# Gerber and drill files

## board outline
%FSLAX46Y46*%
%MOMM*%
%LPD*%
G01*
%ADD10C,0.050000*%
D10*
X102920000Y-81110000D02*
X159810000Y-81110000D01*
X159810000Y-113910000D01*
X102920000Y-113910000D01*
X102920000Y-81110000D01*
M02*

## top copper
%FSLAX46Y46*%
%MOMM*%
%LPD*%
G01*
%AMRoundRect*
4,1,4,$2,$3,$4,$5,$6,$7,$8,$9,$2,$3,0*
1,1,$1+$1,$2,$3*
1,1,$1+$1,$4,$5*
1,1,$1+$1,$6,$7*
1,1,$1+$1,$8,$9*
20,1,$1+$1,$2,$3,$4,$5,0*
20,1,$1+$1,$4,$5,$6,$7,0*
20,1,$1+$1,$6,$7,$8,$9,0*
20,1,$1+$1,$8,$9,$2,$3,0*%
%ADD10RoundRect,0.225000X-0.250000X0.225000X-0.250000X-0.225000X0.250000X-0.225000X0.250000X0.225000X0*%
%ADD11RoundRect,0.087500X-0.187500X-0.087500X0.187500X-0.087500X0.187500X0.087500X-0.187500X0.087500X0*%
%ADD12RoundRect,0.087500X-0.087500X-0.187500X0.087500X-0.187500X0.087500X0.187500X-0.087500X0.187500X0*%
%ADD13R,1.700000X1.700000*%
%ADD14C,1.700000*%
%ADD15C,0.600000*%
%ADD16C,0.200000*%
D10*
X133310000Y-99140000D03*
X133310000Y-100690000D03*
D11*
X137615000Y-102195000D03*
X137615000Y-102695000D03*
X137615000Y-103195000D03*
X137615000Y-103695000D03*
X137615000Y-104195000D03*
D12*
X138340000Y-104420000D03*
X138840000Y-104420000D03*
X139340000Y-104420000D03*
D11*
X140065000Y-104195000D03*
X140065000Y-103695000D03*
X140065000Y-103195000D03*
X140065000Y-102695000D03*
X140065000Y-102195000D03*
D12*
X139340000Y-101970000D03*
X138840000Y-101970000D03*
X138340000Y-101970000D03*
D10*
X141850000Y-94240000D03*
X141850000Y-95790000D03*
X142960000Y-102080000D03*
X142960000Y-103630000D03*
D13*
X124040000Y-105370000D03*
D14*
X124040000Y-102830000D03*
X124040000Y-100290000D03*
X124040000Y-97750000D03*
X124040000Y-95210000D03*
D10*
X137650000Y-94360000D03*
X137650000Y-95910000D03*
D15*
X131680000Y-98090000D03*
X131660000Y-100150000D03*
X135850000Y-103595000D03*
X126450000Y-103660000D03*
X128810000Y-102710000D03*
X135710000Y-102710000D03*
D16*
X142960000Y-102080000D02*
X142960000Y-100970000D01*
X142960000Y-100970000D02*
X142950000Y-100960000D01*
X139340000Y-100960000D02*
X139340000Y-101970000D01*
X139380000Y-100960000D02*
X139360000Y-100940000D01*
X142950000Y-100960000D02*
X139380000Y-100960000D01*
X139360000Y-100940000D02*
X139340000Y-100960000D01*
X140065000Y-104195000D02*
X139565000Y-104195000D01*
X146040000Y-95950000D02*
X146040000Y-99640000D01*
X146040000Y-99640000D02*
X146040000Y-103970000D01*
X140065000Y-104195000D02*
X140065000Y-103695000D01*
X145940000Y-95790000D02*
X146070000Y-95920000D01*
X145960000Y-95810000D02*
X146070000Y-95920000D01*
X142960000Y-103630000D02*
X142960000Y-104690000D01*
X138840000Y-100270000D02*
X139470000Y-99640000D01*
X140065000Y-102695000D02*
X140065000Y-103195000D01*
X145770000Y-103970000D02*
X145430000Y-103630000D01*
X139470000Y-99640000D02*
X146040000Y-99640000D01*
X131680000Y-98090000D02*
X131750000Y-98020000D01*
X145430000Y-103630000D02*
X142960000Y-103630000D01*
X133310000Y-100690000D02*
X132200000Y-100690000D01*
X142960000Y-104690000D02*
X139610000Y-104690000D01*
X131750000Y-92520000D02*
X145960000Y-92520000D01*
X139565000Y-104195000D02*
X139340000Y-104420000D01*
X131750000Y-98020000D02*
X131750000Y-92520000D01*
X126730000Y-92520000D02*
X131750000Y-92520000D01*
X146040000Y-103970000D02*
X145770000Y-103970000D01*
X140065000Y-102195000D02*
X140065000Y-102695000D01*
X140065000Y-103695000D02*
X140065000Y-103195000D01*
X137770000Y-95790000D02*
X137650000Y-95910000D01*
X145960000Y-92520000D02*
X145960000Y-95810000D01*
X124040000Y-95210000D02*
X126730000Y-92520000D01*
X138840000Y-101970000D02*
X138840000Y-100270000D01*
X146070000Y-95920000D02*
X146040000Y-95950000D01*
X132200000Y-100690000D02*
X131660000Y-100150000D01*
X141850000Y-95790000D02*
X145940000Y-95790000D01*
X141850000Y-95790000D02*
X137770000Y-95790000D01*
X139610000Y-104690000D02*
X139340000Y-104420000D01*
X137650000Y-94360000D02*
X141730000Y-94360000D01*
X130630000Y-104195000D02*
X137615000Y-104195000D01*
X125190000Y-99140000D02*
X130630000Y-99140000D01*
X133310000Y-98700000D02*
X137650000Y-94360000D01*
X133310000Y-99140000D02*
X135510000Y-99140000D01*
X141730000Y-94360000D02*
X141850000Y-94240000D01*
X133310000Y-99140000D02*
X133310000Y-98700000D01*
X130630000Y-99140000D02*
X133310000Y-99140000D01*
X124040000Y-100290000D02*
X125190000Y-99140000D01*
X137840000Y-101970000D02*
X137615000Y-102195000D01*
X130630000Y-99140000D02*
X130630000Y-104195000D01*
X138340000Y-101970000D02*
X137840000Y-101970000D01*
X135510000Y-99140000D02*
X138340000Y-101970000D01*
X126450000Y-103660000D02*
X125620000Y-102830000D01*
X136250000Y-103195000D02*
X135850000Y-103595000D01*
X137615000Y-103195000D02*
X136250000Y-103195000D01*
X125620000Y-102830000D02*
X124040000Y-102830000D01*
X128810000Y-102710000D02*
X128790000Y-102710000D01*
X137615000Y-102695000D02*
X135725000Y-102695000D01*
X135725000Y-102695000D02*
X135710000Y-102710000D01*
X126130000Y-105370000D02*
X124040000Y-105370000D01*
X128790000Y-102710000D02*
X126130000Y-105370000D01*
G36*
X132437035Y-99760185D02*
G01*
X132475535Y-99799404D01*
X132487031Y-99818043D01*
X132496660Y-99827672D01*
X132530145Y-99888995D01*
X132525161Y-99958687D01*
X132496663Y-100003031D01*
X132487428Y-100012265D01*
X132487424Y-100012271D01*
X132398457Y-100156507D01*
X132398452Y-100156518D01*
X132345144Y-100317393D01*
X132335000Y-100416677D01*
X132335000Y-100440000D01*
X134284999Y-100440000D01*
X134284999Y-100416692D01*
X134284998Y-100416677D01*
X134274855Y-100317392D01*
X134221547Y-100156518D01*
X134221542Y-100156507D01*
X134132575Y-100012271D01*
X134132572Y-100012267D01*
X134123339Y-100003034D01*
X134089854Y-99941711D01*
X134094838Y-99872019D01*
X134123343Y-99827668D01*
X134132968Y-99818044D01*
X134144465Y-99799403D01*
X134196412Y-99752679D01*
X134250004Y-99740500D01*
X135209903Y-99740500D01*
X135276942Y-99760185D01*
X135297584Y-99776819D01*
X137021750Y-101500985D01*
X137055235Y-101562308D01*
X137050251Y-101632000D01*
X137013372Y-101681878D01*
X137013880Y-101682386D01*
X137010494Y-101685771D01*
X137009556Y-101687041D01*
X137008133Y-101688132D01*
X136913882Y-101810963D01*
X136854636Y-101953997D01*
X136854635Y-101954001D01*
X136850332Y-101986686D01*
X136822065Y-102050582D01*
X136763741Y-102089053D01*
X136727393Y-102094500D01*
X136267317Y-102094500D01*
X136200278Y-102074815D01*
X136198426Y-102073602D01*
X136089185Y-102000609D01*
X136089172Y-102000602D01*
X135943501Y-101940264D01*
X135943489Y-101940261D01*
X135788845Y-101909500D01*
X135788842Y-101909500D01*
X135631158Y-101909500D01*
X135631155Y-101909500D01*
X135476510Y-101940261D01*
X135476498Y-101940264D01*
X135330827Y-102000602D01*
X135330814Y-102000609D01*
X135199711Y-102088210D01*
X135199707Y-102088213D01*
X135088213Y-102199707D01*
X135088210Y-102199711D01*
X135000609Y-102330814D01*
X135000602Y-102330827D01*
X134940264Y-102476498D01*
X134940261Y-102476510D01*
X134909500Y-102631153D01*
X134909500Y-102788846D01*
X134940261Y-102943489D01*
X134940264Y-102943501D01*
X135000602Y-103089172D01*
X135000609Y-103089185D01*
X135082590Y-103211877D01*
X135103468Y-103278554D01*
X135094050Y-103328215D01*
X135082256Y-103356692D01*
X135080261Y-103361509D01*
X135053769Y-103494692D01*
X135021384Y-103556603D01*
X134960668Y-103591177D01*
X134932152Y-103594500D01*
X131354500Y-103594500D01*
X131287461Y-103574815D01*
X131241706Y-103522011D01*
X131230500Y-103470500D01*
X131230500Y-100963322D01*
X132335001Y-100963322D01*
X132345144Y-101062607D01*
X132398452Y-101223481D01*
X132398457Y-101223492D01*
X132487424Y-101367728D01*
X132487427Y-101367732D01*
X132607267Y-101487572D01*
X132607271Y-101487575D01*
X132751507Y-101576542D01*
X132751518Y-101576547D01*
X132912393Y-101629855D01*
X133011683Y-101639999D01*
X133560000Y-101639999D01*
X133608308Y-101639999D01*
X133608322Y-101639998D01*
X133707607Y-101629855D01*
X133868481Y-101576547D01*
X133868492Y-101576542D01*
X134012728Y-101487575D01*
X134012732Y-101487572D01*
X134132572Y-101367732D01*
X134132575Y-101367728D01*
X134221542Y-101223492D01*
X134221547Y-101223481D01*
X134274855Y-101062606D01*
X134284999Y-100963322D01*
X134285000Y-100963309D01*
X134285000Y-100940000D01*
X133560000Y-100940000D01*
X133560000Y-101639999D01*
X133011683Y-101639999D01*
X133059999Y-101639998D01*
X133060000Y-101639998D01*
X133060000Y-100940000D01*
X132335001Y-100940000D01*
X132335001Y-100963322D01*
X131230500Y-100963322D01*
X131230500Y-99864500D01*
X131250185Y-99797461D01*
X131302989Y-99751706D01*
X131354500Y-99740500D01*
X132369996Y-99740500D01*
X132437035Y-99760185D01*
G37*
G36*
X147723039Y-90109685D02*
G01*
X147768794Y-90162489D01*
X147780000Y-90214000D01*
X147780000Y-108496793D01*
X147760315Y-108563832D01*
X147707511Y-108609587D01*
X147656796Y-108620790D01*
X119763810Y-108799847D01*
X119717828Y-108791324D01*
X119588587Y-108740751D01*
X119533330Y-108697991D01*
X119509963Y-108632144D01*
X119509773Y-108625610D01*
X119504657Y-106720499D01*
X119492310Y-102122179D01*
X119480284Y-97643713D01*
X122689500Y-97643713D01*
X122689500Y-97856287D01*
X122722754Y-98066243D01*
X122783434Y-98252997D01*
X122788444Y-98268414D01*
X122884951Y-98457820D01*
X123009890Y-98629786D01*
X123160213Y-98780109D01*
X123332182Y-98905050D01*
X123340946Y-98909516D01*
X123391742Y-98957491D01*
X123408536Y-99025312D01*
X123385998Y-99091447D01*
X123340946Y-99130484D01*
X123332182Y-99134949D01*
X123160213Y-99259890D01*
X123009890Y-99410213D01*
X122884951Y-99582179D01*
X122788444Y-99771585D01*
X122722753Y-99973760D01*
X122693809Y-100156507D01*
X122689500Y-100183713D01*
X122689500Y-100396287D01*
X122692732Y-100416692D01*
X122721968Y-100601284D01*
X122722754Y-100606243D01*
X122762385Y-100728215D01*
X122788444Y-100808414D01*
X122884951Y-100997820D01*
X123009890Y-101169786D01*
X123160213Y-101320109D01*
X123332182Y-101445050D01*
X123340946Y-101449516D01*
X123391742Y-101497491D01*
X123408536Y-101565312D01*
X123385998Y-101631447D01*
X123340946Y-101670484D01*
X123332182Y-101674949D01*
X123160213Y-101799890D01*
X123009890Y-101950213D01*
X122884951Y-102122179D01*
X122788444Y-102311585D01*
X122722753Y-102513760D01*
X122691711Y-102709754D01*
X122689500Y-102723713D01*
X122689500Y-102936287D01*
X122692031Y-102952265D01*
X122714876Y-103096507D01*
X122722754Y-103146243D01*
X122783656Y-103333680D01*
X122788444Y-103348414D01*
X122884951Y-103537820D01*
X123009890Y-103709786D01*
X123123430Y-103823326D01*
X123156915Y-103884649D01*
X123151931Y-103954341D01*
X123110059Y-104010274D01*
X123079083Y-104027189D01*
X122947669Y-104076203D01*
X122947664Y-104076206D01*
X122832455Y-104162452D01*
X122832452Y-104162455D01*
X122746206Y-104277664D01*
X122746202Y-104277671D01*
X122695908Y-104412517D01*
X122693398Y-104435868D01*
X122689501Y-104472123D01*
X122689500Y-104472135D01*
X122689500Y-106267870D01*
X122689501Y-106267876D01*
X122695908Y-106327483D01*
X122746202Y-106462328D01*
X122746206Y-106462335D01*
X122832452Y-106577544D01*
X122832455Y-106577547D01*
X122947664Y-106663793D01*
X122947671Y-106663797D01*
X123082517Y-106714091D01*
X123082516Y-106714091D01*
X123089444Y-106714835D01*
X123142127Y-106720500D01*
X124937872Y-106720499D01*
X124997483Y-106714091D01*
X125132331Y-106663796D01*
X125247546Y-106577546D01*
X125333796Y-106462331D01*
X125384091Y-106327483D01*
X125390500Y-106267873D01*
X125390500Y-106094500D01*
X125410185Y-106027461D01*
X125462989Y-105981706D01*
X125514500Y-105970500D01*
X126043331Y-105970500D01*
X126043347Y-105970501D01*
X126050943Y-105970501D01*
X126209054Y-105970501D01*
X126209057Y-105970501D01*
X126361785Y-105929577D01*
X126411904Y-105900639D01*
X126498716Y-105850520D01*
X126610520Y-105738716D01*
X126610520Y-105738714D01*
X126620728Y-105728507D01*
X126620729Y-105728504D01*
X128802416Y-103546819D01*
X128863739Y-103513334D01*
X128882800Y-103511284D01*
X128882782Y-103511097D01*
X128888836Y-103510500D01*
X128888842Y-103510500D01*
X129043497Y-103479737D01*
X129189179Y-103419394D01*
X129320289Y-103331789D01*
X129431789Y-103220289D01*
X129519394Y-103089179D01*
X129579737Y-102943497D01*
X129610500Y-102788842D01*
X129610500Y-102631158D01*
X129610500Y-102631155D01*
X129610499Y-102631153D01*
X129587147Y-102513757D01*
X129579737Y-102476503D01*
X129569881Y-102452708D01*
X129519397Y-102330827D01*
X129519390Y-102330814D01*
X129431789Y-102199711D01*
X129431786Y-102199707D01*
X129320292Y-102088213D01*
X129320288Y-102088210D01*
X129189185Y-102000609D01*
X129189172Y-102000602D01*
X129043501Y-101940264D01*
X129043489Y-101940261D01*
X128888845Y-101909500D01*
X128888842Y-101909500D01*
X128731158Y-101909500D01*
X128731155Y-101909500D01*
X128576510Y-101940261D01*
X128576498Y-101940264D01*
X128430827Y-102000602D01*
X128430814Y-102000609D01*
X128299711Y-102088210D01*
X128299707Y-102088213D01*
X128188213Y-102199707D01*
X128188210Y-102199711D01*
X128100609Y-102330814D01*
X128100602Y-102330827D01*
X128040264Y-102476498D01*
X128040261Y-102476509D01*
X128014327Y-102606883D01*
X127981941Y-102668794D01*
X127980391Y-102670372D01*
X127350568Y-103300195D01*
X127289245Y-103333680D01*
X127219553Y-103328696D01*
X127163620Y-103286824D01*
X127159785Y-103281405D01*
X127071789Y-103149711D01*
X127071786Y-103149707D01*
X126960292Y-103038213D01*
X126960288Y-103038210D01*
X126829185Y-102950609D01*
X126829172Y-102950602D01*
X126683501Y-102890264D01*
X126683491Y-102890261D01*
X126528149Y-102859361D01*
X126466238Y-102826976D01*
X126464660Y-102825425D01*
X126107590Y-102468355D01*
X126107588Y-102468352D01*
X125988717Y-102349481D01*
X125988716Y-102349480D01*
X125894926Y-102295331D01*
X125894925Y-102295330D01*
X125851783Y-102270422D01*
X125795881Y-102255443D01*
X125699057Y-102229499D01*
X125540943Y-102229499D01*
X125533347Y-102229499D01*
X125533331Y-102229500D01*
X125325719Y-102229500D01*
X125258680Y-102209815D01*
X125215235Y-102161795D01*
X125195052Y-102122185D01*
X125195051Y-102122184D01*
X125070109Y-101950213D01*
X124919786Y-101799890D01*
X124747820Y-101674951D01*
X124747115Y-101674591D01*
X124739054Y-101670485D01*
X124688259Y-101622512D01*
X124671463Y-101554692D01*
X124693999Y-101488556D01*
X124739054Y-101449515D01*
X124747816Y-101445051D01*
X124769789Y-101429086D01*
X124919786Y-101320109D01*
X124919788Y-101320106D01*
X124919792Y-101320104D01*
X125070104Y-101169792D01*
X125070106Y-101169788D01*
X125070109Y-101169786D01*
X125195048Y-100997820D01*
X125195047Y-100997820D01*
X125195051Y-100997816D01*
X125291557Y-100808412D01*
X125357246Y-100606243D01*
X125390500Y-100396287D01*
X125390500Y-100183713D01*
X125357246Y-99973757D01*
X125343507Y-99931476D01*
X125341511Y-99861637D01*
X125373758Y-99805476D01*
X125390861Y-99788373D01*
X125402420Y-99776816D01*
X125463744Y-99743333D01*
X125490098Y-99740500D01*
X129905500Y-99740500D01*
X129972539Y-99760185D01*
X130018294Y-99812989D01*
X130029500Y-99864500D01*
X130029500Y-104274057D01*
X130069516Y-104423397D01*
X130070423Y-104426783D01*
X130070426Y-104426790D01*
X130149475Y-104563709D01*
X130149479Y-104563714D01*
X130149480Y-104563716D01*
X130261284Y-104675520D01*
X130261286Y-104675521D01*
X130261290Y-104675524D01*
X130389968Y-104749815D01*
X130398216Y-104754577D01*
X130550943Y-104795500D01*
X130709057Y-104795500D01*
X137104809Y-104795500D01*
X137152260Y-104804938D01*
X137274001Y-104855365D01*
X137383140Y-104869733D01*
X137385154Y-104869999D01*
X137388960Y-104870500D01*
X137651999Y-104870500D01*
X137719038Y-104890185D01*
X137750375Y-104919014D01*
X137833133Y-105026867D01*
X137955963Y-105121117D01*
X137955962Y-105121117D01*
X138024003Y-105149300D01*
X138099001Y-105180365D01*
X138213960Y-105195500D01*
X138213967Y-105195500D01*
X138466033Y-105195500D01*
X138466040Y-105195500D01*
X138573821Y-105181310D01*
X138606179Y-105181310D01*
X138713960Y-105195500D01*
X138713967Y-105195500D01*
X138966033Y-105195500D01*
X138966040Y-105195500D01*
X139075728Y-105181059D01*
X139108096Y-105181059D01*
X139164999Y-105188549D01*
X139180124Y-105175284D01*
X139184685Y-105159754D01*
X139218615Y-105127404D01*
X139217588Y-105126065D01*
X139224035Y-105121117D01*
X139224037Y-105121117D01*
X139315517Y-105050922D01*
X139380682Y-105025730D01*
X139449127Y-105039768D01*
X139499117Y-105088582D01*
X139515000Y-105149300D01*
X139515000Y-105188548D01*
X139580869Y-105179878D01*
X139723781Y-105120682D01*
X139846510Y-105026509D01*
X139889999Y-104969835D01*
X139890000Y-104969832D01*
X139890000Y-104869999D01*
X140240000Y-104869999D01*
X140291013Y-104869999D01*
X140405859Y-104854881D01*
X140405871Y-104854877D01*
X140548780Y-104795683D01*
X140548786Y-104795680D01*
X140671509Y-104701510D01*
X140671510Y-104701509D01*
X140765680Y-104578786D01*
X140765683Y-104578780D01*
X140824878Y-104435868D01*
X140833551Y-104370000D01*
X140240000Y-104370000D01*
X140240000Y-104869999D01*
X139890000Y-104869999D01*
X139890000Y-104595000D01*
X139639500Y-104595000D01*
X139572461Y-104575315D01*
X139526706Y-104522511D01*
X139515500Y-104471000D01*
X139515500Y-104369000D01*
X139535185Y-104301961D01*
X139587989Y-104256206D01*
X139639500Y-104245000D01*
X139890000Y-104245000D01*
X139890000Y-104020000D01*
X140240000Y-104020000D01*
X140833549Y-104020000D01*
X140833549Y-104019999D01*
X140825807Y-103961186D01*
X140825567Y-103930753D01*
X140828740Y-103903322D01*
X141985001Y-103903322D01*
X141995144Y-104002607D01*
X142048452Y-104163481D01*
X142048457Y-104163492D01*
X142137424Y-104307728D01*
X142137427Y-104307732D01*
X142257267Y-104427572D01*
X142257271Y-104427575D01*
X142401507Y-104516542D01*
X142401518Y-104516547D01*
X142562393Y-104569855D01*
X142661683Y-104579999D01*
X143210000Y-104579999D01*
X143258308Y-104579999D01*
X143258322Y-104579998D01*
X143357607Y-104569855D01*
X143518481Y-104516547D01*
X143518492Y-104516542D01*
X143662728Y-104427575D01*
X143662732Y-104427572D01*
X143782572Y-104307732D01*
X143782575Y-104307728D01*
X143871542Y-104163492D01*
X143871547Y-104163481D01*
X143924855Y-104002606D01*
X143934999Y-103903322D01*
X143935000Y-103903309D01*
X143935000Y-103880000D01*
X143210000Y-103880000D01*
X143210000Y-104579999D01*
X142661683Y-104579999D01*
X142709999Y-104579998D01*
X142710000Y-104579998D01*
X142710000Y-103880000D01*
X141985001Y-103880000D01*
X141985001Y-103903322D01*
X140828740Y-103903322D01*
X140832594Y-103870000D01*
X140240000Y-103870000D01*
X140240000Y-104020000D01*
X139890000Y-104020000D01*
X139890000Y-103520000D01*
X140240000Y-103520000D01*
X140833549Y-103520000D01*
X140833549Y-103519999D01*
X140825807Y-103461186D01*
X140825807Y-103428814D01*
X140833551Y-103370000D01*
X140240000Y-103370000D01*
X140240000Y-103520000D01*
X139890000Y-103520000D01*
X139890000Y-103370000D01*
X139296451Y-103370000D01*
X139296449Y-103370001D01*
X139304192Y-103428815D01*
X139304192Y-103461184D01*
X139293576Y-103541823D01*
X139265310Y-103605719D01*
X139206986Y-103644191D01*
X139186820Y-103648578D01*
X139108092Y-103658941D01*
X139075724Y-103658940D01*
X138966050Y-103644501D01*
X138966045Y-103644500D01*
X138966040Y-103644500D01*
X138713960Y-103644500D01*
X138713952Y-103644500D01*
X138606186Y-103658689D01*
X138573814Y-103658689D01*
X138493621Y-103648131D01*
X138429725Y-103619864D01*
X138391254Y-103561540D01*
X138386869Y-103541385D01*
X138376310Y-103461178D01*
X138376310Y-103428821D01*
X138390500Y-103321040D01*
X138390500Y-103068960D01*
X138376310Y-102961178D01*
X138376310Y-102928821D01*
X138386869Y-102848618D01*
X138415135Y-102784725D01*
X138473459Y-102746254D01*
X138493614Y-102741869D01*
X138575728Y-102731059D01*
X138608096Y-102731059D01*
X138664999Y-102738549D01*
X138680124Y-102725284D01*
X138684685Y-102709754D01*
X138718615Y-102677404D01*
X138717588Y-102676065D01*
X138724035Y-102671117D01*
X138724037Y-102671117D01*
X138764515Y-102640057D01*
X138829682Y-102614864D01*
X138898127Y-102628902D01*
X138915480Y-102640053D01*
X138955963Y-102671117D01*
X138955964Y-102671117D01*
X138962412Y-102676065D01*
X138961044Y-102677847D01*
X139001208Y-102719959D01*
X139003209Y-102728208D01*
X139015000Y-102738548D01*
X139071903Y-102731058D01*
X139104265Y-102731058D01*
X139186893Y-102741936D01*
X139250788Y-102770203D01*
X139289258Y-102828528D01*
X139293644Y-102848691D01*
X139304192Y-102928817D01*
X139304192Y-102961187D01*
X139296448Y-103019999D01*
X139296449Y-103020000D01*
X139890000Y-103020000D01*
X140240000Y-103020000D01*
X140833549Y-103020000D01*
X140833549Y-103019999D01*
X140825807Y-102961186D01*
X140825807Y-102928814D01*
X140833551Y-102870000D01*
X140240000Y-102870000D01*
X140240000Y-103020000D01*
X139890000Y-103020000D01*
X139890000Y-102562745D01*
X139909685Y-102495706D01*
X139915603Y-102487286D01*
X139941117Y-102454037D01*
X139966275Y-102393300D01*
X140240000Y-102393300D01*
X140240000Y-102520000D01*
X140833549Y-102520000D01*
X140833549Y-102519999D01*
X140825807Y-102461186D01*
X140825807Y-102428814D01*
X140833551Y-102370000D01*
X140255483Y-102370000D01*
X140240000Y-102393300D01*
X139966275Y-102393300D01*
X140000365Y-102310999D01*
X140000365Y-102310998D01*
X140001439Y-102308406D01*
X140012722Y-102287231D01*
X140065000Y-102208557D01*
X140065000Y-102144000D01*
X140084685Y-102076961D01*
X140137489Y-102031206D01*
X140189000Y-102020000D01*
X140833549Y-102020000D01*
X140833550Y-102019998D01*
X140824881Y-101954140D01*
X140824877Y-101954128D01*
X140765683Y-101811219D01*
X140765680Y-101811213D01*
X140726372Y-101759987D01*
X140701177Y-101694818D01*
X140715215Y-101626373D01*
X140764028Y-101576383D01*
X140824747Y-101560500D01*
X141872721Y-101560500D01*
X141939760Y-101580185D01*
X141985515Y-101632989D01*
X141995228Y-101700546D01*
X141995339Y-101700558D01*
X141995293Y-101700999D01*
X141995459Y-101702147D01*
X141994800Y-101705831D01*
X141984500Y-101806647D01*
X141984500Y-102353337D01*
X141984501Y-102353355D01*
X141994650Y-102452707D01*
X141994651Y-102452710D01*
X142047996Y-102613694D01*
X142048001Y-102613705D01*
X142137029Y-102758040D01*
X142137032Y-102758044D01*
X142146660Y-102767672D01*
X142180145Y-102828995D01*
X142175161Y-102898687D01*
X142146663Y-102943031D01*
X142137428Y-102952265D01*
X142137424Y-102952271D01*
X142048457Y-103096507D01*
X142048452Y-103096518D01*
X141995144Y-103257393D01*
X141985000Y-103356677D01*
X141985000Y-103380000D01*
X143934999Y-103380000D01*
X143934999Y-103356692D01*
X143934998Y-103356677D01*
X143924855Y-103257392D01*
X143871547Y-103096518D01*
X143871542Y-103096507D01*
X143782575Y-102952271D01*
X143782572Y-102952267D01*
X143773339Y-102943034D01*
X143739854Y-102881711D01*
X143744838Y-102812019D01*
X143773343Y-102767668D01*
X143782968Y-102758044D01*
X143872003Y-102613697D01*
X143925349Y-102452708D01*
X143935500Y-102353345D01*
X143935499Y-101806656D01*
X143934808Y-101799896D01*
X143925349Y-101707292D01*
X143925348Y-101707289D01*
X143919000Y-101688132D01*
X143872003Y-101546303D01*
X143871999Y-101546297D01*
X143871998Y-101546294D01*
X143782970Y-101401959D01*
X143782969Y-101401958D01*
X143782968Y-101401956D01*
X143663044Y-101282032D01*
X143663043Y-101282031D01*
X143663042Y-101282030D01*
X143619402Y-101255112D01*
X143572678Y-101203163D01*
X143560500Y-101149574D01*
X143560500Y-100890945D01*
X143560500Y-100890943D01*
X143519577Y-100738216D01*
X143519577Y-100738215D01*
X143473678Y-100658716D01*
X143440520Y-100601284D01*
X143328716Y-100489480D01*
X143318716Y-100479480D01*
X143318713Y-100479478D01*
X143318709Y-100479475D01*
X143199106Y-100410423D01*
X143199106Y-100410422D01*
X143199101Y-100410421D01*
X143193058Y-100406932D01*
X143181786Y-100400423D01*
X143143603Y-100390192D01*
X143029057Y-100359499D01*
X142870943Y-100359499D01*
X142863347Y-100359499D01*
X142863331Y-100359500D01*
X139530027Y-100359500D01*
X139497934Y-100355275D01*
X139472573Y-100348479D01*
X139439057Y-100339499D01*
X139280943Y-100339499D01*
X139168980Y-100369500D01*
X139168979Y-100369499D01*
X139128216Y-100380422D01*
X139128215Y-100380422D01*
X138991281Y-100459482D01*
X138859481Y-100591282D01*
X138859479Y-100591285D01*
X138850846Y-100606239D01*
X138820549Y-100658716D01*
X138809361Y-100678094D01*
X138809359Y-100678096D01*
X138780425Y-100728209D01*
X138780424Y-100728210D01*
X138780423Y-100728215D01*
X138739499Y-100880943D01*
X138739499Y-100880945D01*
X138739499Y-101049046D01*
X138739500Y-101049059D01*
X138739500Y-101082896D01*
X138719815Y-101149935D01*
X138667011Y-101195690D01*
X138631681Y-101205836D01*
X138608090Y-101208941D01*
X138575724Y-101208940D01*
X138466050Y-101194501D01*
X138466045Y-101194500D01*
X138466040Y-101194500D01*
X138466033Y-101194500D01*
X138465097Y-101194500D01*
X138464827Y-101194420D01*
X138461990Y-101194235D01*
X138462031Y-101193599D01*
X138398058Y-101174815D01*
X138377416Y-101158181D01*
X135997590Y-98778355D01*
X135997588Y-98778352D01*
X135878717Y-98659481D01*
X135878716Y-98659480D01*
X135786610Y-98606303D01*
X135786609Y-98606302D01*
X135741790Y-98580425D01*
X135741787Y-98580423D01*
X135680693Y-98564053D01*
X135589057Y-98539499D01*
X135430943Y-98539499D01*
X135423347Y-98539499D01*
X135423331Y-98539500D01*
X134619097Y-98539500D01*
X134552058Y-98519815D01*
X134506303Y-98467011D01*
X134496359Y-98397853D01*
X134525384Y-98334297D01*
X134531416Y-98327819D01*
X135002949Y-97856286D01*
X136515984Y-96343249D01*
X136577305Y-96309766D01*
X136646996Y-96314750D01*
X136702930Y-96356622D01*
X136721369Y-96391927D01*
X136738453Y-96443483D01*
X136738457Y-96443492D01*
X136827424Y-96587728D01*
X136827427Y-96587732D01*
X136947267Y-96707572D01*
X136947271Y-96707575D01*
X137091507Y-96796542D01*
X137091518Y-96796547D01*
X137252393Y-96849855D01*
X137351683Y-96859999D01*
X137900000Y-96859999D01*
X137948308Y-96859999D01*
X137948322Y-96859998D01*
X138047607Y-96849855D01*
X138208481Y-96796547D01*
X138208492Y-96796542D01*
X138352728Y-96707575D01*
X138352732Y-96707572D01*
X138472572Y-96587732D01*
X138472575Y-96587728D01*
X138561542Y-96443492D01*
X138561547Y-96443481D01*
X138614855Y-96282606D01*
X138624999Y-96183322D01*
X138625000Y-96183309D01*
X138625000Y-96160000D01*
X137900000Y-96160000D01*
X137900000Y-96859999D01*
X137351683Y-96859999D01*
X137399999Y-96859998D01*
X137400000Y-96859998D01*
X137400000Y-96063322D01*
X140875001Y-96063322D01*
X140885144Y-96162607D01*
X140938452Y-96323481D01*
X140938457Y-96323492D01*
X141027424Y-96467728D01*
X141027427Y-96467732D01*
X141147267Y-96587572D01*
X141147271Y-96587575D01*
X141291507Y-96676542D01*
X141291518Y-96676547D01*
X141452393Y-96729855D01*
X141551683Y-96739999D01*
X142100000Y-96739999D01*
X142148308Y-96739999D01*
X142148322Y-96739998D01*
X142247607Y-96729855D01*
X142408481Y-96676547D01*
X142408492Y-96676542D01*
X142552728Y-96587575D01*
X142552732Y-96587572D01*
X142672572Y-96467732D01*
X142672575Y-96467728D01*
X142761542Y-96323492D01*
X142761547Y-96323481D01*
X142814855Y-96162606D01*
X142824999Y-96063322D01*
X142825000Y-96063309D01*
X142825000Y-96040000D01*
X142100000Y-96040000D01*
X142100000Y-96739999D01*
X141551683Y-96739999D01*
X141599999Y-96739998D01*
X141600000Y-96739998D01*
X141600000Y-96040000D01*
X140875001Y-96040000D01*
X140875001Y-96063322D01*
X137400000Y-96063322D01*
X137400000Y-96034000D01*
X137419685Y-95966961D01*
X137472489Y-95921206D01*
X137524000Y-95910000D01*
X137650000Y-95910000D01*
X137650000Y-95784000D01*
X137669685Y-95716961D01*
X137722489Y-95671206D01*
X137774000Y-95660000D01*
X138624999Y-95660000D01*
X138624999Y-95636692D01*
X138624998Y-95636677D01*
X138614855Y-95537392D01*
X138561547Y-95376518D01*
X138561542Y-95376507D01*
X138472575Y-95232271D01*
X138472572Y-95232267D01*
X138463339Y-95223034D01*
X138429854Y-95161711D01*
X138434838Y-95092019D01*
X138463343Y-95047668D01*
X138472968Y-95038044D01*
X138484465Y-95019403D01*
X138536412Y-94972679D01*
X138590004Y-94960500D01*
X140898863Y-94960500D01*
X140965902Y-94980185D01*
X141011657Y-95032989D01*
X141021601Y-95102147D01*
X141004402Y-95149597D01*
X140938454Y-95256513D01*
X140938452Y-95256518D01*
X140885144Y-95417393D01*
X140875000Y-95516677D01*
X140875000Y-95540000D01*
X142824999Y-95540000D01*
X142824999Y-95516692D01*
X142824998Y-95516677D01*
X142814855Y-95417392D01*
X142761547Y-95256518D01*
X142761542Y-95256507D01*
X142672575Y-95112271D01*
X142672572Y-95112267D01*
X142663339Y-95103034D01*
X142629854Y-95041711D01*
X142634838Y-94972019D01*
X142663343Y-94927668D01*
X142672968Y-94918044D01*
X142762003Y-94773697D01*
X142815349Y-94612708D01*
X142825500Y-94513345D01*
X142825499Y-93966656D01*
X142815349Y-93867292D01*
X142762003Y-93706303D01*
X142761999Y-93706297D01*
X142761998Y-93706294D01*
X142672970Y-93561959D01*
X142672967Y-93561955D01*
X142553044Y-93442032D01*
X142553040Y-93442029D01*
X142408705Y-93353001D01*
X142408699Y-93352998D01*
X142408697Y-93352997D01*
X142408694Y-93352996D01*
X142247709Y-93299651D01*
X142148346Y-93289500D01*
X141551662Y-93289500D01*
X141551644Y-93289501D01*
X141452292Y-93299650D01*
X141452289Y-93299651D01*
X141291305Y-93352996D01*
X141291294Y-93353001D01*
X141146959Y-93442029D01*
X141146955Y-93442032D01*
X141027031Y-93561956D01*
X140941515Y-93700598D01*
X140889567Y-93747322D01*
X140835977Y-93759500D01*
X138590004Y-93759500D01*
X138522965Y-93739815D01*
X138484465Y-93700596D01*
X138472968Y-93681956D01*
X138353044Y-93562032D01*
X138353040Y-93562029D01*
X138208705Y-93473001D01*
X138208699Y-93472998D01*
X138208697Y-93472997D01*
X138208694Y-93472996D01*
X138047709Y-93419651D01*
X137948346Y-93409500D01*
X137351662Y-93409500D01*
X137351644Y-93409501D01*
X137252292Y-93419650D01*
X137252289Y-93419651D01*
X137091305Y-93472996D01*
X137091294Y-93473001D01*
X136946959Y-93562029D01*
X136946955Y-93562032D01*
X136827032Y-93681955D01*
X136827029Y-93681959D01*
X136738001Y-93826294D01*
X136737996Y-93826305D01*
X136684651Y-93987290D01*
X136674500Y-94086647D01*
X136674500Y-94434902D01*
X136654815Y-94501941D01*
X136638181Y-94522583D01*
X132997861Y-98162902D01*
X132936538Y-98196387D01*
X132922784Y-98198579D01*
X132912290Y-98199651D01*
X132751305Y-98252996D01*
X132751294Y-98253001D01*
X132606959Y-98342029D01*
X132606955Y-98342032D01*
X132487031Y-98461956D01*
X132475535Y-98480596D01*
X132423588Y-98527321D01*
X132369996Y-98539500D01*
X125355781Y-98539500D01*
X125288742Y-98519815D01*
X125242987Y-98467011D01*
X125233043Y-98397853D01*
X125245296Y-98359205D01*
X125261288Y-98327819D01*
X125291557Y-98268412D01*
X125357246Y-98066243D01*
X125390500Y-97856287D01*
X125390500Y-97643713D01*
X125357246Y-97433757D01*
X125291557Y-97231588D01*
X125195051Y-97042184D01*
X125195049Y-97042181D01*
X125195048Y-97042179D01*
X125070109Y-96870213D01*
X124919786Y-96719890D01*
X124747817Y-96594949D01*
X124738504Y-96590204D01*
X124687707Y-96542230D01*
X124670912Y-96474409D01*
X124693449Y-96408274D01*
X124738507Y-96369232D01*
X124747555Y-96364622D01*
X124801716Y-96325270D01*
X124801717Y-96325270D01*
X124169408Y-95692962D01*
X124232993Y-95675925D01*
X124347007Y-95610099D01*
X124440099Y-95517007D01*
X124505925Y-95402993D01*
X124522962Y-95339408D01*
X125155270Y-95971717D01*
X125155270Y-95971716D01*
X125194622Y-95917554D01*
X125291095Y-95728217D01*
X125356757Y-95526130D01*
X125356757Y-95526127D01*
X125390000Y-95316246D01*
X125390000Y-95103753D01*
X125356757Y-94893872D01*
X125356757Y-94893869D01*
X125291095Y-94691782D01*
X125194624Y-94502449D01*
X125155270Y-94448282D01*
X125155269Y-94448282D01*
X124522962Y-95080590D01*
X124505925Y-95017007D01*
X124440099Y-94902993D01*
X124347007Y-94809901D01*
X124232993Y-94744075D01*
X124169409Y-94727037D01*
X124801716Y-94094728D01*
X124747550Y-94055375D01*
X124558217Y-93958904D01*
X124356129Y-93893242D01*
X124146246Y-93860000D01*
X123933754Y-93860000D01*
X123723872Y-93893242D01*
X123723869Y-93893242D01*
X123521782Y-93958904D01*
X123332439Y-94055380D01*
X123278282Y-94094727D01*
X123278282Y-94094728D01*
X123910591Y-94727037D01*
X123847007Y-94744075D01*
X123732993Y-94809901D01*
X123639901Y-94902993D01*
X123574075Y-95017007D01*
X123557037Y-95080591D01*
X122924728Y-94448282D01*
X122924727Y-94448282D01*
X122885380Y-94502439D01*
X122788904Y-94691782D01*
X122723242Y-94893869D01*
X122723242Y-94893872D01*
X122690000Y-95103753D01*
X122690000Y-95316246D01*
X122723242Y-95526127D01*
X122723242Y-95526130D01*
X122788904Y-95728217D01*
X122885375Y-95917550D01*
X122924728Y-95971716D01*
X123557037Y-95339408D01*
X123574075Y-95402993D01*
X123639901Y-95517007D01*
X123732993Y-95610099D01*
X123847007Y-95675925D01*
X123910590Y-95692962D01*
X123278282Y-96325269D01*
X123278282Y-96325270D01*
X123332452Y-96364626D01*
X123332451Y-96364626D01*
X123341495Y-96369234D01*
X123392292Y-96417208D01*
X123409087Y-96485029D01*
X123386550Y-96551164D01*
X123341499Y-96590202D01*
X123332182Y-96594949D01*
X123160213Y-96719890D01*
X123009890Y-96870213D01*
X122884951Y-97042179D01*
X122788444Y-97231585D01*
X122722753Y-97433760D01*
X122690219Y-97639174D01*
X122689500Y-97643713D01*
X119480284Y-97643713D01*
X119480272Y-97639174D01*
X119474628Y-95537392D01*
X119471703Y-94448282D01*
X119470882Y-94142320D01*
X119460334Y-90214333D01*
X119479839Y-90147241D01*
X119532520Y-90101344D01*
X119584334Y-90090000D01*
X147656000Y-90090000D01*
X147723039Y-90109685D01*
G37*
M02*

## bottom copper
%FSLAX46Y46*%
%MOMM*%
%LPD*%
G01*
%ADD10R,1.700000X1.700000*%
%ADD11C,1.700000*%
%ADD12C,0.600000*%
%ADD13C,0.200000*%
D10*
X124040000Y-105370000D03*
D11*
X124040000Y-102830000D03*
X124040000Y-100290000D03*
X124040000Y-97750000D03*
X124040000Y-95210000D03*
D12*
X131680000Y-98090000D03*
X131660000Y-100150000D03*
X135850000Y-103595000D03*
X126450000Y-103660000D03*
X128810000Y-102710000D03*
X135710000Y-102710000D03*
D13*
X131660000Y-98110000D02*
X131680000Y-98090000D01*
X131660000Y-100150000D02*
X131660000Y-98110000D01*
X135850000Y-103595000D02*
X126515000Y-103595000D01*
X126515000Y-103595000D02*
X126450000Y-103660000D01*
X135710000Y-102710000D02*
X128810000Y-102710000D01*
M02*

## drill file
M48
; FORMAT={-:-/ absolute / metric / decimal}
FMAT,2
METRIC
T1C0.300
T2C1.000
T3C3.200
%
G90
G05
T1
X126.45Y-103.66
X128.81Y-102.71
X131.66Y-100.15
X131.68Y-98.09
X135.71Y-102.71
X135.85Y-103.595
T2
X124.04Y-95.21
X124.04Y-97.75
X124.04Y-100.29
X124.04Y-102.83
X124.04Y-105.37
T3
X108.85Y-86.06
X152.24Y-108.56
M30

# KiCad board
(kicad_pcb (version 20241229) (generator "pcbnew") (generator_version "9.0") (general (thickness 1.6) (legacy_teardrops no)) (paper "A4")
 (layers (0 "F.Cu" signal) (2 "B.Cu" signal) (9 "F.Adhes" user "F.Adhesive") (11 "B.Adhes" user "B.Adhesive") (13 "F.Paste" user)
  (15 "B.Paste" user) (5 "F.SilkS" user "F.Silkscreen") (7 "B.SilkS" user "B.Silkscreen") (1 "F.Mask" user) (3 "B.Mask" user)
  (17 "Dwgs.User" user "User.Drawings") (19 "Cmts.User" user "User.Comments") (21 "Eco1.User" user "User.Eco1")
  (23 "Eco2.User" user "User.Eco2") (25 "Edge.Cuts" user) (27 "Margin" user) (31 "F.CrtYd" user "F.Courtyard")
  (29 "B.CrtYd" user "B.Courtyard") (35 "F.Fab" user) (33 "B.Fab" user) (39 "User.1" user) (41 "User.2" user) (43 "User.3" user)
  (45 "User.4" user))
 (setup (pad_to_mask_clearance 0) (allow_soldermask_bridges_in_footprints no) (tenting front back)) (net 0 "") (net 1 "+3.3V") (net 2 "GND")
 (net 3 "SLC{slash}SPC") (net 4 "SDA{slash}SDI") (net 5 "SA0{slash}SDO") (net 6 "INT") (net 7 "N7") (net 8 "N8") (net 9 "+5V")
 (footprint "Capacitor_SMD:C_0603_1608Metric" (layer "F.Cu") (at 133.31 99.915 -90)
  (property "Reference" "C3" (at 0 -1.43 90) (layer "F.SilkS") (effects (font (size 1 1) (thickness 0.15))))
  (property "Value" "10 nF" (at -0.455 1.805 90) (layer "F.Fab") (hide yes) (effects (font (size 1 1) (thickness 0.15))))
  (pad "1" smd roundrect (at -0.775 0 270) (size 0.9 0.95) (layers "F.Cu" "F.Mask" "F.Paste") (roundrect_rratio 0.25) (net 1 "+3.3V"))
  (pad "2" smd roundrect (at 0.775 0 270) (size 0.9 0.95) (layers "F.Cu" "F.Mask" "F.Paste") (roundrect_rratio 0.25) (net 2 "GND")))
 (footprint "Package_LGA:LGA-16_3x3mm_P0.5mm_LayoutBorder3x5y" (layer "F.Cu") (at 138.84 103.195)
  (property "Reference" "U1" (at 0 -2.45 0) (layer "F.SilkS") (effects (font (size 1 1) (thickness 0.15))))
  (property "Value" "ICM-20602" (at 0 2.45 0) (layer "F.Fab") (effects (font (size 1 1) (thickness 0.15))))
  (pad "1" smd roundrect (at -1.225 -1) (size 0.55 0.35) (layers "F.Cu" "F.Mask" "F.Paste") (roundrect_rratio 0.25) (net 1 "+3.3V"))
  (pad "2" smd roundrect (at -1.225 -0.5) (size 0.55 0.35) (layers "F.Cu" "F.Mask" "F.Paste") (roundrect_rratio 0.25)
   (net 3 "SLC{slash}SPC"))
  (pad "3" smd roundrect (at -1.225 0) (size 0.55 0.35) (layers "F.Cu" "F.Mask" "F.Paste") (roundrect_rratio 0.25) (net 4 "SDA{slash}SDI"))
  (pad "4" smd roundrect (at -1.225 0.5) (size 0.55 0.35) (layers "F.Cu" "F.Mask" "F.Paste") (roundrect_rratio 0.25) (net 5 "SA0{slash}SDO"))
  (pad "5" smd roundrect (at -1.225 1) (size 0.55 0.35) (layers "F.Cu" "F.Mask" "F.Paste") (roundrect_rratio 0.25) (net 1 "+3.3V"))
  (pad "6" smd roundrect (at -0.5 1.225) (size 0.35 0.55) (layers "F.Cu" "F.Mask" "F.Paste") (roundrect_rratio 0.25) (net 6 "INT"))
  (pad "7" smd roundrect (at 0 1.225) (size 0.35 0.55) (layers "F.Cu" "F.Mask" "F.Paste") (roundrect_rratio 0.25) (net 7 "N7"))
  (pad "8" smd roundrect (at 0.5 1.225) (size 0.35 0.55) (layers "F.Cu" "F.Mask" "F.Paste") (roundrect_rratio 0.25) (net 2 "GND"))
  (pad "9" smd roundrect (at 1.225 1) (size 0.55 0.35) (layers "F.Cu" "F.Mask" "F.Paste") (roundrect_rratio 0.25) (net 2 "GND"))
  (pad "10" smd roundrect (at 1.225 0.5) (size 0.55 0.35) (layers "F.Cu" "F.Mask" "F.Paste") (roundrect_rratio 0.25) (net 2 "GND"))
  (pad "11" smd roundrect (at 1.225 0) (size 0.55 0.35) (layers "F.Cu" "F.Mask" "F.Paste") (roundrect_rratio 0.25) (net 2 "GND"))
  (pad "12" smd roundrect (at 1.225 -0.5) (size 0.55 0.35) (layers "F.Cu" "F.Mask" "F.Paste") (roundrect_rratio 0.25) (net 2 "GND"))
  (pad "13" smd roundrect (at 1.225 -1) (size 0.55 0.35) (layers "F.Cu" "F.Mask" "F.Paste") (roundrect_rratio 0.25) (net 2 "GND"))
  (pad "14" smd roundrect (at 0.5 -1.225) (size 0.35 0.55) (layers "F.Cu" "F.Mask" "F.Paste") (roundrect_rratio 0.25) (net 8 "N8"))
  (pad "15" smd roundrect (at 0 -1.225) (size 0.35 0.55) (layers "F.Cu" "F.Mask" "F.Paste") (roundrect_rratio 0.25) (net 2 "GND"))
  (pad "16" smd roundrect (at -0.5 -1.225) (size 0.35 0.55) (layers "F.Cu" "F.Mask" "F.Paste") (roundrect_rratio 0.25) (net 1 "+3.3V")))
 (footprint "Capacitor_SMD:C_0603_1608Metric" (layer "F.Cu") (at 141.85 95.015 -90)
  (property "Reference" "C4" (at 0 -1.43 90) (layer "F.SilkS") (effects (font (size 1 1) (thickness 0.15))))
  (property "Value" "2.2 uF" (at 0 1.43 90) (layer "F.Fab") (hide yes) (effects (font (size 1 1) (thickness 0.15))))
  (pad "1" smd roundrect (at -0.775 0 270) (size 0.9 0.95) (layers "F.Cu" "F.Mask" "F.Paste") (roundrect_rratio 0.25) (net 1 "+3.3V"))
  (pad "2" smd roundrect (at 0.775 0 270) (size 0.9 0.95) (layers "F.Cu" "F.Mask" "F.Paste") (roundrect_rratio 0.25) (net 2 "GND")))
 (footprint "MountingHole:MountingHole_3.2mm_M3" (layer "F.Cu") (at 108.85 86.06)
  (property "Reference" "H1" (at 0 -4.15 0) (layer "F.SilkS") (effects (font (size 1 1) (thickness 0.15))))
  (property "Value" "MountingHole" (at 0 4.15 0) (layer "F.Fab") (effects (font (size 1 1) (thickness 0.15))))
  (pad "" np_thru_hole circle (at 0 0) (size 3.2 3.2) (drill 3.2) (layers "*.Cu" "*.Mask")))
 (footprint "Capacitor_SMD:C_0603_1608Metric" (layer "F.Cu") (at 142.96 102.855 -90)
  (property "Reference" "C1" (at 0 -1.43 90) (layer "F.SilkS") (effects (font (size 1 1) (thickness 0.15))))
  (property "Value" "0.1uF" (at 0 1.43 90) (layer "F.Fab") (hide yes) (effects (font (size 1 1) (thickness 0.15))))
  (pad "1" smd roundrect (at -0.775 0 270) (size 0.9 0.95) (layers "F.Cu" "F.Mask" "F.Paste") (roundrect_rratio 0.25) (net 8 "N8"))
  (pad "2" smd roundrect (at 0.775 0 270) (size 0.9 0.95) (layers "F.Cu" "F.Mask" "F.Paste") (roundrect_rratio 0.25) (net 2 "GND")))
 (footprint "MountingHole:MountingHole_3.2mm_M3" (layer "F.Cu") (at 152.24 108.56)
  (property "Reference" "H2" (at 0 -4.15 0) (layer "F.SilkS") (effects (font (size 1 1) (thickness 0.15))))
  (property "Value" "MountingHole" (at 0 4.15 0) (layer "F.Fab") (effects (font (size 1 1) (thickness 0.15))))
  (pad "" np_thru_hole circle (at 0 0) (size 3.2 3.2) (drill 3.2) (layers "*.Cu" "*.Mask")))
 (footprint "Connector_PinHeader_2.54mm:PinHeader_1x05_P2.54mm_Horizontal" (layer "F.Cu") (at 124.04 105.37 180)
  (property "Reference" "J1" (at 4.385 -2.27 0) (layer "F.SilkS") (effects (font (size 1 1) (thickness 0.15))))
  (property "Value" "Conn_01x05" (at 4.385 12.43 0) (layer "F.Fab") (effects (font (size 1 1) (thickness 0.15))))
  (pad "1" thru_hole rect (at 0 0 180) (size 1.7 1.7) (drill 1) (layers "*.Cu" "*.Mask") (remove_unused_layers no) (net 3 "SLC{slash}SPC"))
  (pad "2" thru_hole circle (at 0 2.54 180) (size 1.7 1.7) (drill 1) (layers "*.Cu" "*.Mask") (remove_unused_layers no)
   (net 4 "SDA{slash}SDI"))
  (pad "3" thru_hole circle (at 0 5.08 180) (size 1.7 1.7) (drill 1) (layers "*.Cu" "*.Mask") (remove_unused_layers no) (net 1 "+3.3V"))
  (pad "4" thru_hole circle (at 0 7.62 180) (size 1.7 1.7) (drill 1) (layers "*.Cu" "*.Mask") (remove_unused_layers no) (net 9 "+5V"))
  (pad "5" thru_hole circle (at 0 10.16 180) (size 1.7 1.7) (drill 1) (layers "*.Cu" "*.Mask") (remove_unused_layers no) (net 2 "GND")))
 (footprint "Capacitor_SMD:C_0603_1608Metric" (layer "F.Cu") (at 137.65 95.135 -90)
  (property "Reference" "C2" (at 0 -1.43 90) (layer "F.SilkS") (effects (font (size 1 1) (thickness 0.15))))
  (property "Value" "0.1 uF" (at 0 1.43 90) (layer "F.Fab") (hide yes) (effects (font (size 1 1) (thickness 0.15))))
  (pad "1" smd roundrect (at -0.775 0 270) (size 0.9 0.95) (layers "F.Cu" "F.Mask" "F.Paste") (roundrect_rratio 0.25) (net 1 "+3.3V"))
  (pad "2" smd roundrect (at 0.775 0 270) (size 0.9 0.95) (layers "F.Cu" "F.Mask" "F.Paste") (roundrect_rratio 0.25) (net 2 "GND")))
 (gr_rect (start 102.92 81.11) (end 159.81 113.91) (stroke (width 0.05) (type default)) (fill no) (layer "Edge.Cuts"))
 (segment (start 142.96 102.08) (end 142.96 100.97) (width 0.2) (layer "F.Cu") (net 8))
 (segment (start 142.96 100.97) (end 142.95 100.96) (width 0.2) (layer "F.Cu") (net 8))
 (segment (start 139.34 100.96) (end 139.34 101.97) (width 0.2) (layer "F.Cu") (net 8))
 (segment (start 139.38 100.96) (end 139.36 100.94) (width 0.2) (layer "F.Cu") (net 8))
 (segment (start 142.95 100.96) (end 139.38 100.96) (width 0.2) (layer "F.Cu") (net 8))
 (segment (start 139.36 100.94) (end 139.34 100.96) (width 0.2) (layer "F.Cu") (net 8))
 (segment (start 140.065 104.195) (end 139.565 104.195) (width 0.2) (layer "F.Cu") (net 2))
 (segment (start 146.04 95.95) (end 146.04 99.64) (width 0.2) (layer "F.Cu") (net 2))
 (segment (start 146.04 99.64) (end 146.04 103.97) (width 0.2) (layer "F.Cu") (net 2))
 (segment (start 140.065 104.195) (end 140.065 103.695) (width 0.2) (layer "F.Cu") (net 2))
 (segment (start 145.94 95.79) (end 146.07 95.92) (width 0.2) (layer "F.Cu") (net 2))
 (segment (start 145.96 95.81) (end 146.07 95.92) (width 0.2) (layer "F.Cu") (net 2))
 (segment (start 142.96 103.63) (end 142.96 104.69) (width 0.2) (layer "F.Cu") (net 2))
 (segment (start 138.84 100.27) (end 139.47 99.64) (width 0.2) (layer "F.Cu") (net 2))
 (segment (start 140.065 102.695) (end 140.065 103.195) (width 0.2) (layer "F.Cu") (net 2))
 (segment (start 145.77 103.97) (end 145.43 103.63) (width 0.2) (layer "F.Cu") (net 2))
 (segment (start 139.47 99.64) (end 146.04 99.64) (width 0.2) (layer "F.Cu") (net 2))
 (segment (start 131.68 98.09) (end 131.75 98.02) (width 0.2) (layer "F.Cu") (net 2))
 (segment (start 145.43 103.63) (end 142.96 103.63) (width 0.2) (layer "F.Cu") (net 2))
 (segment (start 133.31 100.69) (end 132.2 100.69) (width 0.2) (layer "F.Cu") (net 2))
 (segment (start 142.96 104.69) (end 139.61 104.69) (width 0.2) (layer "F.Cu") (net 2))
 (segment (start 131.75 92.52) (end 145.96 92.52) (width 0.2) (layer "F.Cu") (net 2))
 (segment (start 139.565 104.195) (end 139.34 104.42) (width 0.2) (layer "F.Cu") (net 2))
 (segment (start 131.75 98.02) (end 131.75 92.52) (width 0.2) (layer "F.Cu") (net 2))
 (segment (start 126.73 92.52) (end 131.75 92.52) (width 0.2) (layer "F.Cu") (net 2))
 (segment (start 146.04 103.97) (end 145.77 103.97) (width 0.2) (layer "F.Cu") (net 2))
 (segment (start 140.065 102.195) (end 140.065 102.695) (width 0.2) (layer "F.Cu") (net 2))
 (segment (start 140.065 103.695) (end 140.065 103.195) (width 0.2) (layer "F.Cu") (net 2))
 (segment (start 137.77 95.79) (end 137.65 95.91) (width 0.2) (layer "F.Cu") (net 2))
 (segment (start 145.96 92.52) (end 145.96 95.81) (width 0.2) (layer "F.Cu") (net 2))
 (segment (start 124.04 95.21) (end 126.73 92.52) (width 0.2) (layer "F.Cu") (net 2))
 (segment (start 138.84 101.97) (end 138.84 100.27) (width 0.2) (layer "F.Cu") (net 2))
 (segment (start 146.07 95.92) (end 146.04 95.95) (width 0.2) (layer "F.Cu") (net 2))
 (segment (start 132.2 100.69) (end 131.66 100.15) (width 0.2) (layer "F.Cu") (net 2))
 (segment (start 141.85 95.79) (end 145.94 95.79) (width 0.2) (layer "F.Cu") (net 2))
 (segment (start 141.85 95.79) (end 137.77 95.79) (width 0.2) (layer "F.Cu") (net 2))
 (segment (start 139.61 104.69) (end 139.34 104.42) (width 0.2) (layer "F.Cu") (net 2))
 (via (at 131.68 98.09) (size 0.6) (drill 0.3) (layers "F.Cu" "B.Cu") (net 2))
 (via (at 131.66 100.15) (size 0.6) (drill 0.3) (layers "F.Cu" "B.Cu") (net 2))
 (segment (start 131.66 98.11) (end 131.68 98.09) (width 0.2) (layer "B.Cu") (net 2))
 (segment (start 131.66 100.15) (end 131.66 98.11) (width 0.2) (layer "B.Cu") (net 2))
 (segment (start 137.65 94.36) (end 141.73 94.36) (width 0.2) (layer "F.Cu") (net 1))
 (segment (start 130.63 104.195) (end 137.615 104.195) (width 0.2) (layer "F.Cu") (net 1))
 (segment (start 125.19 99.14) (end 130.63 99.14) (width 0.2) (layer "F.Cu") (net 1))
 (segment (start 133.31 98.7) (end 137.65 94.36) (width 0.2) (layer "F.Cu") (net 1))
 (segment (start 133.31 99.14) (end 135.51 99.14) (width 0.2) (layer "F.Cu") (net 1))
 (segment (start 141.73 94.36) (end 141.85 94.24) (width 0.2) (layer "F.Cu") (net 1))
 (segment (start 133.31 99.14) (end 133.31 98.7) (width 0.2) (layer "F.Cu") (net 1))
 (segment (start 130.63 99.14) (end 133.31 99.14) (width 0.2) (layer "F.Cu") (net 1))
 (segment (start 124.04 100.29) (end 125.19 99.14) (width 0.2) (layer "F.Cu") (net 1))
 (segment (start 137.84 101.97) (end 137.615 102.195) (width 0.2) (layer "F.Cu") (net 1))
 (segment (start 130.63 99.14) (end 130.63 104.195) (width 0.2) (layer "F.Cu") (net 1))
 (segment (start 138.34 101.97) (end 137.84 101.97) (width 0.2) (layer "F.Cu") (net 1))
 (segment (start 135.51 99.14) (end 138.34 101.97) (width 0.2) (layer "F.Cu") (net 1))
 (segment (start 126.45 103.66) (end 125.62 102.83) (width 0.2) (layer "F.Cu") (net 4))
 (segment (start 136.25 103.195) (end 135.85 103.595) (width 0.2) (layer "F.Cu") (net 4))
 (segment (start 137.615 103.195) (end 136.25 103.195) (width 0.2) (layer "F.Cu") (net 4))
 (segment (start 125.62 102.83) (end 124.04 102.83) (width 0.2) (layer "F.Cu") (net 4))
 (via (at 135.85 103.595) (size 0.6) (drill 0.3) (layers "F.Cu" "B.Cu") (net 4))
 (via (at 126.45 103.66) (size 0.6) (drill 0.3) (layers "F.Cu" "B.Cu") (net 4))
 (segment (start 135.85 103.595) (end 126.515 103.595) (width 0.2) (layer "B.Cu") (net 4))
 (segment (start 126.515 103.595) (end 126.45 103.66) (width 0.2) (layer "B.Cu") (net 4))
 (segment (start 128.81 102.71) (end 128.79 102.71) (width 0.2) (layer "F.Cu") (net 3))
 (segment (start 137.615 102.695) (end 135.725 102.695) (width 0.2) (layer "F.Cu") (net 3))
 (segment (start 135.725 102.695) (end 135.71 102.71) (width 0.2) (layer "F.Cu") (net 3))
 (segment (start 126.13 105.37) (end 124.04 105.37) (width 0.2) (layer "F.Cu") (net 3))
 (segment (start 128.79 102.71) (end 126.13 105.37) (width 0.2) (layer "F.Cu") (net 3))
 (via (at 128.81 102.71) (size 0.6) (drill 0.3) (layers "F.Cu" "B.Cu") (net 3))
 (via (at 135.71 102.71) (size 0.6) (drill 0.3) (layers "F.Cu" "B.Cu") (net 3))
 (segment (start 135.71 102.71) (end 128.81 102.71) (width 0.2) (layer "B.Cu") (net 3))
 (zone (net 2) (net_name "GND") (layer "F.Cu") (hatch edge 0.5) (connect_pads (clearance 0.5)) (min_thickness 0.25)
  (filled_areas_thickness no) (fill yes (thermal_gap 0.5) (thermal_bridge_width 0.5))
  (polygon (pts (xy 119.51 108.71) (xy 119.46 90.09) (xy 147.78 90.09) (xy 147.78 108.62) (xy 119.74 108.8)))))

